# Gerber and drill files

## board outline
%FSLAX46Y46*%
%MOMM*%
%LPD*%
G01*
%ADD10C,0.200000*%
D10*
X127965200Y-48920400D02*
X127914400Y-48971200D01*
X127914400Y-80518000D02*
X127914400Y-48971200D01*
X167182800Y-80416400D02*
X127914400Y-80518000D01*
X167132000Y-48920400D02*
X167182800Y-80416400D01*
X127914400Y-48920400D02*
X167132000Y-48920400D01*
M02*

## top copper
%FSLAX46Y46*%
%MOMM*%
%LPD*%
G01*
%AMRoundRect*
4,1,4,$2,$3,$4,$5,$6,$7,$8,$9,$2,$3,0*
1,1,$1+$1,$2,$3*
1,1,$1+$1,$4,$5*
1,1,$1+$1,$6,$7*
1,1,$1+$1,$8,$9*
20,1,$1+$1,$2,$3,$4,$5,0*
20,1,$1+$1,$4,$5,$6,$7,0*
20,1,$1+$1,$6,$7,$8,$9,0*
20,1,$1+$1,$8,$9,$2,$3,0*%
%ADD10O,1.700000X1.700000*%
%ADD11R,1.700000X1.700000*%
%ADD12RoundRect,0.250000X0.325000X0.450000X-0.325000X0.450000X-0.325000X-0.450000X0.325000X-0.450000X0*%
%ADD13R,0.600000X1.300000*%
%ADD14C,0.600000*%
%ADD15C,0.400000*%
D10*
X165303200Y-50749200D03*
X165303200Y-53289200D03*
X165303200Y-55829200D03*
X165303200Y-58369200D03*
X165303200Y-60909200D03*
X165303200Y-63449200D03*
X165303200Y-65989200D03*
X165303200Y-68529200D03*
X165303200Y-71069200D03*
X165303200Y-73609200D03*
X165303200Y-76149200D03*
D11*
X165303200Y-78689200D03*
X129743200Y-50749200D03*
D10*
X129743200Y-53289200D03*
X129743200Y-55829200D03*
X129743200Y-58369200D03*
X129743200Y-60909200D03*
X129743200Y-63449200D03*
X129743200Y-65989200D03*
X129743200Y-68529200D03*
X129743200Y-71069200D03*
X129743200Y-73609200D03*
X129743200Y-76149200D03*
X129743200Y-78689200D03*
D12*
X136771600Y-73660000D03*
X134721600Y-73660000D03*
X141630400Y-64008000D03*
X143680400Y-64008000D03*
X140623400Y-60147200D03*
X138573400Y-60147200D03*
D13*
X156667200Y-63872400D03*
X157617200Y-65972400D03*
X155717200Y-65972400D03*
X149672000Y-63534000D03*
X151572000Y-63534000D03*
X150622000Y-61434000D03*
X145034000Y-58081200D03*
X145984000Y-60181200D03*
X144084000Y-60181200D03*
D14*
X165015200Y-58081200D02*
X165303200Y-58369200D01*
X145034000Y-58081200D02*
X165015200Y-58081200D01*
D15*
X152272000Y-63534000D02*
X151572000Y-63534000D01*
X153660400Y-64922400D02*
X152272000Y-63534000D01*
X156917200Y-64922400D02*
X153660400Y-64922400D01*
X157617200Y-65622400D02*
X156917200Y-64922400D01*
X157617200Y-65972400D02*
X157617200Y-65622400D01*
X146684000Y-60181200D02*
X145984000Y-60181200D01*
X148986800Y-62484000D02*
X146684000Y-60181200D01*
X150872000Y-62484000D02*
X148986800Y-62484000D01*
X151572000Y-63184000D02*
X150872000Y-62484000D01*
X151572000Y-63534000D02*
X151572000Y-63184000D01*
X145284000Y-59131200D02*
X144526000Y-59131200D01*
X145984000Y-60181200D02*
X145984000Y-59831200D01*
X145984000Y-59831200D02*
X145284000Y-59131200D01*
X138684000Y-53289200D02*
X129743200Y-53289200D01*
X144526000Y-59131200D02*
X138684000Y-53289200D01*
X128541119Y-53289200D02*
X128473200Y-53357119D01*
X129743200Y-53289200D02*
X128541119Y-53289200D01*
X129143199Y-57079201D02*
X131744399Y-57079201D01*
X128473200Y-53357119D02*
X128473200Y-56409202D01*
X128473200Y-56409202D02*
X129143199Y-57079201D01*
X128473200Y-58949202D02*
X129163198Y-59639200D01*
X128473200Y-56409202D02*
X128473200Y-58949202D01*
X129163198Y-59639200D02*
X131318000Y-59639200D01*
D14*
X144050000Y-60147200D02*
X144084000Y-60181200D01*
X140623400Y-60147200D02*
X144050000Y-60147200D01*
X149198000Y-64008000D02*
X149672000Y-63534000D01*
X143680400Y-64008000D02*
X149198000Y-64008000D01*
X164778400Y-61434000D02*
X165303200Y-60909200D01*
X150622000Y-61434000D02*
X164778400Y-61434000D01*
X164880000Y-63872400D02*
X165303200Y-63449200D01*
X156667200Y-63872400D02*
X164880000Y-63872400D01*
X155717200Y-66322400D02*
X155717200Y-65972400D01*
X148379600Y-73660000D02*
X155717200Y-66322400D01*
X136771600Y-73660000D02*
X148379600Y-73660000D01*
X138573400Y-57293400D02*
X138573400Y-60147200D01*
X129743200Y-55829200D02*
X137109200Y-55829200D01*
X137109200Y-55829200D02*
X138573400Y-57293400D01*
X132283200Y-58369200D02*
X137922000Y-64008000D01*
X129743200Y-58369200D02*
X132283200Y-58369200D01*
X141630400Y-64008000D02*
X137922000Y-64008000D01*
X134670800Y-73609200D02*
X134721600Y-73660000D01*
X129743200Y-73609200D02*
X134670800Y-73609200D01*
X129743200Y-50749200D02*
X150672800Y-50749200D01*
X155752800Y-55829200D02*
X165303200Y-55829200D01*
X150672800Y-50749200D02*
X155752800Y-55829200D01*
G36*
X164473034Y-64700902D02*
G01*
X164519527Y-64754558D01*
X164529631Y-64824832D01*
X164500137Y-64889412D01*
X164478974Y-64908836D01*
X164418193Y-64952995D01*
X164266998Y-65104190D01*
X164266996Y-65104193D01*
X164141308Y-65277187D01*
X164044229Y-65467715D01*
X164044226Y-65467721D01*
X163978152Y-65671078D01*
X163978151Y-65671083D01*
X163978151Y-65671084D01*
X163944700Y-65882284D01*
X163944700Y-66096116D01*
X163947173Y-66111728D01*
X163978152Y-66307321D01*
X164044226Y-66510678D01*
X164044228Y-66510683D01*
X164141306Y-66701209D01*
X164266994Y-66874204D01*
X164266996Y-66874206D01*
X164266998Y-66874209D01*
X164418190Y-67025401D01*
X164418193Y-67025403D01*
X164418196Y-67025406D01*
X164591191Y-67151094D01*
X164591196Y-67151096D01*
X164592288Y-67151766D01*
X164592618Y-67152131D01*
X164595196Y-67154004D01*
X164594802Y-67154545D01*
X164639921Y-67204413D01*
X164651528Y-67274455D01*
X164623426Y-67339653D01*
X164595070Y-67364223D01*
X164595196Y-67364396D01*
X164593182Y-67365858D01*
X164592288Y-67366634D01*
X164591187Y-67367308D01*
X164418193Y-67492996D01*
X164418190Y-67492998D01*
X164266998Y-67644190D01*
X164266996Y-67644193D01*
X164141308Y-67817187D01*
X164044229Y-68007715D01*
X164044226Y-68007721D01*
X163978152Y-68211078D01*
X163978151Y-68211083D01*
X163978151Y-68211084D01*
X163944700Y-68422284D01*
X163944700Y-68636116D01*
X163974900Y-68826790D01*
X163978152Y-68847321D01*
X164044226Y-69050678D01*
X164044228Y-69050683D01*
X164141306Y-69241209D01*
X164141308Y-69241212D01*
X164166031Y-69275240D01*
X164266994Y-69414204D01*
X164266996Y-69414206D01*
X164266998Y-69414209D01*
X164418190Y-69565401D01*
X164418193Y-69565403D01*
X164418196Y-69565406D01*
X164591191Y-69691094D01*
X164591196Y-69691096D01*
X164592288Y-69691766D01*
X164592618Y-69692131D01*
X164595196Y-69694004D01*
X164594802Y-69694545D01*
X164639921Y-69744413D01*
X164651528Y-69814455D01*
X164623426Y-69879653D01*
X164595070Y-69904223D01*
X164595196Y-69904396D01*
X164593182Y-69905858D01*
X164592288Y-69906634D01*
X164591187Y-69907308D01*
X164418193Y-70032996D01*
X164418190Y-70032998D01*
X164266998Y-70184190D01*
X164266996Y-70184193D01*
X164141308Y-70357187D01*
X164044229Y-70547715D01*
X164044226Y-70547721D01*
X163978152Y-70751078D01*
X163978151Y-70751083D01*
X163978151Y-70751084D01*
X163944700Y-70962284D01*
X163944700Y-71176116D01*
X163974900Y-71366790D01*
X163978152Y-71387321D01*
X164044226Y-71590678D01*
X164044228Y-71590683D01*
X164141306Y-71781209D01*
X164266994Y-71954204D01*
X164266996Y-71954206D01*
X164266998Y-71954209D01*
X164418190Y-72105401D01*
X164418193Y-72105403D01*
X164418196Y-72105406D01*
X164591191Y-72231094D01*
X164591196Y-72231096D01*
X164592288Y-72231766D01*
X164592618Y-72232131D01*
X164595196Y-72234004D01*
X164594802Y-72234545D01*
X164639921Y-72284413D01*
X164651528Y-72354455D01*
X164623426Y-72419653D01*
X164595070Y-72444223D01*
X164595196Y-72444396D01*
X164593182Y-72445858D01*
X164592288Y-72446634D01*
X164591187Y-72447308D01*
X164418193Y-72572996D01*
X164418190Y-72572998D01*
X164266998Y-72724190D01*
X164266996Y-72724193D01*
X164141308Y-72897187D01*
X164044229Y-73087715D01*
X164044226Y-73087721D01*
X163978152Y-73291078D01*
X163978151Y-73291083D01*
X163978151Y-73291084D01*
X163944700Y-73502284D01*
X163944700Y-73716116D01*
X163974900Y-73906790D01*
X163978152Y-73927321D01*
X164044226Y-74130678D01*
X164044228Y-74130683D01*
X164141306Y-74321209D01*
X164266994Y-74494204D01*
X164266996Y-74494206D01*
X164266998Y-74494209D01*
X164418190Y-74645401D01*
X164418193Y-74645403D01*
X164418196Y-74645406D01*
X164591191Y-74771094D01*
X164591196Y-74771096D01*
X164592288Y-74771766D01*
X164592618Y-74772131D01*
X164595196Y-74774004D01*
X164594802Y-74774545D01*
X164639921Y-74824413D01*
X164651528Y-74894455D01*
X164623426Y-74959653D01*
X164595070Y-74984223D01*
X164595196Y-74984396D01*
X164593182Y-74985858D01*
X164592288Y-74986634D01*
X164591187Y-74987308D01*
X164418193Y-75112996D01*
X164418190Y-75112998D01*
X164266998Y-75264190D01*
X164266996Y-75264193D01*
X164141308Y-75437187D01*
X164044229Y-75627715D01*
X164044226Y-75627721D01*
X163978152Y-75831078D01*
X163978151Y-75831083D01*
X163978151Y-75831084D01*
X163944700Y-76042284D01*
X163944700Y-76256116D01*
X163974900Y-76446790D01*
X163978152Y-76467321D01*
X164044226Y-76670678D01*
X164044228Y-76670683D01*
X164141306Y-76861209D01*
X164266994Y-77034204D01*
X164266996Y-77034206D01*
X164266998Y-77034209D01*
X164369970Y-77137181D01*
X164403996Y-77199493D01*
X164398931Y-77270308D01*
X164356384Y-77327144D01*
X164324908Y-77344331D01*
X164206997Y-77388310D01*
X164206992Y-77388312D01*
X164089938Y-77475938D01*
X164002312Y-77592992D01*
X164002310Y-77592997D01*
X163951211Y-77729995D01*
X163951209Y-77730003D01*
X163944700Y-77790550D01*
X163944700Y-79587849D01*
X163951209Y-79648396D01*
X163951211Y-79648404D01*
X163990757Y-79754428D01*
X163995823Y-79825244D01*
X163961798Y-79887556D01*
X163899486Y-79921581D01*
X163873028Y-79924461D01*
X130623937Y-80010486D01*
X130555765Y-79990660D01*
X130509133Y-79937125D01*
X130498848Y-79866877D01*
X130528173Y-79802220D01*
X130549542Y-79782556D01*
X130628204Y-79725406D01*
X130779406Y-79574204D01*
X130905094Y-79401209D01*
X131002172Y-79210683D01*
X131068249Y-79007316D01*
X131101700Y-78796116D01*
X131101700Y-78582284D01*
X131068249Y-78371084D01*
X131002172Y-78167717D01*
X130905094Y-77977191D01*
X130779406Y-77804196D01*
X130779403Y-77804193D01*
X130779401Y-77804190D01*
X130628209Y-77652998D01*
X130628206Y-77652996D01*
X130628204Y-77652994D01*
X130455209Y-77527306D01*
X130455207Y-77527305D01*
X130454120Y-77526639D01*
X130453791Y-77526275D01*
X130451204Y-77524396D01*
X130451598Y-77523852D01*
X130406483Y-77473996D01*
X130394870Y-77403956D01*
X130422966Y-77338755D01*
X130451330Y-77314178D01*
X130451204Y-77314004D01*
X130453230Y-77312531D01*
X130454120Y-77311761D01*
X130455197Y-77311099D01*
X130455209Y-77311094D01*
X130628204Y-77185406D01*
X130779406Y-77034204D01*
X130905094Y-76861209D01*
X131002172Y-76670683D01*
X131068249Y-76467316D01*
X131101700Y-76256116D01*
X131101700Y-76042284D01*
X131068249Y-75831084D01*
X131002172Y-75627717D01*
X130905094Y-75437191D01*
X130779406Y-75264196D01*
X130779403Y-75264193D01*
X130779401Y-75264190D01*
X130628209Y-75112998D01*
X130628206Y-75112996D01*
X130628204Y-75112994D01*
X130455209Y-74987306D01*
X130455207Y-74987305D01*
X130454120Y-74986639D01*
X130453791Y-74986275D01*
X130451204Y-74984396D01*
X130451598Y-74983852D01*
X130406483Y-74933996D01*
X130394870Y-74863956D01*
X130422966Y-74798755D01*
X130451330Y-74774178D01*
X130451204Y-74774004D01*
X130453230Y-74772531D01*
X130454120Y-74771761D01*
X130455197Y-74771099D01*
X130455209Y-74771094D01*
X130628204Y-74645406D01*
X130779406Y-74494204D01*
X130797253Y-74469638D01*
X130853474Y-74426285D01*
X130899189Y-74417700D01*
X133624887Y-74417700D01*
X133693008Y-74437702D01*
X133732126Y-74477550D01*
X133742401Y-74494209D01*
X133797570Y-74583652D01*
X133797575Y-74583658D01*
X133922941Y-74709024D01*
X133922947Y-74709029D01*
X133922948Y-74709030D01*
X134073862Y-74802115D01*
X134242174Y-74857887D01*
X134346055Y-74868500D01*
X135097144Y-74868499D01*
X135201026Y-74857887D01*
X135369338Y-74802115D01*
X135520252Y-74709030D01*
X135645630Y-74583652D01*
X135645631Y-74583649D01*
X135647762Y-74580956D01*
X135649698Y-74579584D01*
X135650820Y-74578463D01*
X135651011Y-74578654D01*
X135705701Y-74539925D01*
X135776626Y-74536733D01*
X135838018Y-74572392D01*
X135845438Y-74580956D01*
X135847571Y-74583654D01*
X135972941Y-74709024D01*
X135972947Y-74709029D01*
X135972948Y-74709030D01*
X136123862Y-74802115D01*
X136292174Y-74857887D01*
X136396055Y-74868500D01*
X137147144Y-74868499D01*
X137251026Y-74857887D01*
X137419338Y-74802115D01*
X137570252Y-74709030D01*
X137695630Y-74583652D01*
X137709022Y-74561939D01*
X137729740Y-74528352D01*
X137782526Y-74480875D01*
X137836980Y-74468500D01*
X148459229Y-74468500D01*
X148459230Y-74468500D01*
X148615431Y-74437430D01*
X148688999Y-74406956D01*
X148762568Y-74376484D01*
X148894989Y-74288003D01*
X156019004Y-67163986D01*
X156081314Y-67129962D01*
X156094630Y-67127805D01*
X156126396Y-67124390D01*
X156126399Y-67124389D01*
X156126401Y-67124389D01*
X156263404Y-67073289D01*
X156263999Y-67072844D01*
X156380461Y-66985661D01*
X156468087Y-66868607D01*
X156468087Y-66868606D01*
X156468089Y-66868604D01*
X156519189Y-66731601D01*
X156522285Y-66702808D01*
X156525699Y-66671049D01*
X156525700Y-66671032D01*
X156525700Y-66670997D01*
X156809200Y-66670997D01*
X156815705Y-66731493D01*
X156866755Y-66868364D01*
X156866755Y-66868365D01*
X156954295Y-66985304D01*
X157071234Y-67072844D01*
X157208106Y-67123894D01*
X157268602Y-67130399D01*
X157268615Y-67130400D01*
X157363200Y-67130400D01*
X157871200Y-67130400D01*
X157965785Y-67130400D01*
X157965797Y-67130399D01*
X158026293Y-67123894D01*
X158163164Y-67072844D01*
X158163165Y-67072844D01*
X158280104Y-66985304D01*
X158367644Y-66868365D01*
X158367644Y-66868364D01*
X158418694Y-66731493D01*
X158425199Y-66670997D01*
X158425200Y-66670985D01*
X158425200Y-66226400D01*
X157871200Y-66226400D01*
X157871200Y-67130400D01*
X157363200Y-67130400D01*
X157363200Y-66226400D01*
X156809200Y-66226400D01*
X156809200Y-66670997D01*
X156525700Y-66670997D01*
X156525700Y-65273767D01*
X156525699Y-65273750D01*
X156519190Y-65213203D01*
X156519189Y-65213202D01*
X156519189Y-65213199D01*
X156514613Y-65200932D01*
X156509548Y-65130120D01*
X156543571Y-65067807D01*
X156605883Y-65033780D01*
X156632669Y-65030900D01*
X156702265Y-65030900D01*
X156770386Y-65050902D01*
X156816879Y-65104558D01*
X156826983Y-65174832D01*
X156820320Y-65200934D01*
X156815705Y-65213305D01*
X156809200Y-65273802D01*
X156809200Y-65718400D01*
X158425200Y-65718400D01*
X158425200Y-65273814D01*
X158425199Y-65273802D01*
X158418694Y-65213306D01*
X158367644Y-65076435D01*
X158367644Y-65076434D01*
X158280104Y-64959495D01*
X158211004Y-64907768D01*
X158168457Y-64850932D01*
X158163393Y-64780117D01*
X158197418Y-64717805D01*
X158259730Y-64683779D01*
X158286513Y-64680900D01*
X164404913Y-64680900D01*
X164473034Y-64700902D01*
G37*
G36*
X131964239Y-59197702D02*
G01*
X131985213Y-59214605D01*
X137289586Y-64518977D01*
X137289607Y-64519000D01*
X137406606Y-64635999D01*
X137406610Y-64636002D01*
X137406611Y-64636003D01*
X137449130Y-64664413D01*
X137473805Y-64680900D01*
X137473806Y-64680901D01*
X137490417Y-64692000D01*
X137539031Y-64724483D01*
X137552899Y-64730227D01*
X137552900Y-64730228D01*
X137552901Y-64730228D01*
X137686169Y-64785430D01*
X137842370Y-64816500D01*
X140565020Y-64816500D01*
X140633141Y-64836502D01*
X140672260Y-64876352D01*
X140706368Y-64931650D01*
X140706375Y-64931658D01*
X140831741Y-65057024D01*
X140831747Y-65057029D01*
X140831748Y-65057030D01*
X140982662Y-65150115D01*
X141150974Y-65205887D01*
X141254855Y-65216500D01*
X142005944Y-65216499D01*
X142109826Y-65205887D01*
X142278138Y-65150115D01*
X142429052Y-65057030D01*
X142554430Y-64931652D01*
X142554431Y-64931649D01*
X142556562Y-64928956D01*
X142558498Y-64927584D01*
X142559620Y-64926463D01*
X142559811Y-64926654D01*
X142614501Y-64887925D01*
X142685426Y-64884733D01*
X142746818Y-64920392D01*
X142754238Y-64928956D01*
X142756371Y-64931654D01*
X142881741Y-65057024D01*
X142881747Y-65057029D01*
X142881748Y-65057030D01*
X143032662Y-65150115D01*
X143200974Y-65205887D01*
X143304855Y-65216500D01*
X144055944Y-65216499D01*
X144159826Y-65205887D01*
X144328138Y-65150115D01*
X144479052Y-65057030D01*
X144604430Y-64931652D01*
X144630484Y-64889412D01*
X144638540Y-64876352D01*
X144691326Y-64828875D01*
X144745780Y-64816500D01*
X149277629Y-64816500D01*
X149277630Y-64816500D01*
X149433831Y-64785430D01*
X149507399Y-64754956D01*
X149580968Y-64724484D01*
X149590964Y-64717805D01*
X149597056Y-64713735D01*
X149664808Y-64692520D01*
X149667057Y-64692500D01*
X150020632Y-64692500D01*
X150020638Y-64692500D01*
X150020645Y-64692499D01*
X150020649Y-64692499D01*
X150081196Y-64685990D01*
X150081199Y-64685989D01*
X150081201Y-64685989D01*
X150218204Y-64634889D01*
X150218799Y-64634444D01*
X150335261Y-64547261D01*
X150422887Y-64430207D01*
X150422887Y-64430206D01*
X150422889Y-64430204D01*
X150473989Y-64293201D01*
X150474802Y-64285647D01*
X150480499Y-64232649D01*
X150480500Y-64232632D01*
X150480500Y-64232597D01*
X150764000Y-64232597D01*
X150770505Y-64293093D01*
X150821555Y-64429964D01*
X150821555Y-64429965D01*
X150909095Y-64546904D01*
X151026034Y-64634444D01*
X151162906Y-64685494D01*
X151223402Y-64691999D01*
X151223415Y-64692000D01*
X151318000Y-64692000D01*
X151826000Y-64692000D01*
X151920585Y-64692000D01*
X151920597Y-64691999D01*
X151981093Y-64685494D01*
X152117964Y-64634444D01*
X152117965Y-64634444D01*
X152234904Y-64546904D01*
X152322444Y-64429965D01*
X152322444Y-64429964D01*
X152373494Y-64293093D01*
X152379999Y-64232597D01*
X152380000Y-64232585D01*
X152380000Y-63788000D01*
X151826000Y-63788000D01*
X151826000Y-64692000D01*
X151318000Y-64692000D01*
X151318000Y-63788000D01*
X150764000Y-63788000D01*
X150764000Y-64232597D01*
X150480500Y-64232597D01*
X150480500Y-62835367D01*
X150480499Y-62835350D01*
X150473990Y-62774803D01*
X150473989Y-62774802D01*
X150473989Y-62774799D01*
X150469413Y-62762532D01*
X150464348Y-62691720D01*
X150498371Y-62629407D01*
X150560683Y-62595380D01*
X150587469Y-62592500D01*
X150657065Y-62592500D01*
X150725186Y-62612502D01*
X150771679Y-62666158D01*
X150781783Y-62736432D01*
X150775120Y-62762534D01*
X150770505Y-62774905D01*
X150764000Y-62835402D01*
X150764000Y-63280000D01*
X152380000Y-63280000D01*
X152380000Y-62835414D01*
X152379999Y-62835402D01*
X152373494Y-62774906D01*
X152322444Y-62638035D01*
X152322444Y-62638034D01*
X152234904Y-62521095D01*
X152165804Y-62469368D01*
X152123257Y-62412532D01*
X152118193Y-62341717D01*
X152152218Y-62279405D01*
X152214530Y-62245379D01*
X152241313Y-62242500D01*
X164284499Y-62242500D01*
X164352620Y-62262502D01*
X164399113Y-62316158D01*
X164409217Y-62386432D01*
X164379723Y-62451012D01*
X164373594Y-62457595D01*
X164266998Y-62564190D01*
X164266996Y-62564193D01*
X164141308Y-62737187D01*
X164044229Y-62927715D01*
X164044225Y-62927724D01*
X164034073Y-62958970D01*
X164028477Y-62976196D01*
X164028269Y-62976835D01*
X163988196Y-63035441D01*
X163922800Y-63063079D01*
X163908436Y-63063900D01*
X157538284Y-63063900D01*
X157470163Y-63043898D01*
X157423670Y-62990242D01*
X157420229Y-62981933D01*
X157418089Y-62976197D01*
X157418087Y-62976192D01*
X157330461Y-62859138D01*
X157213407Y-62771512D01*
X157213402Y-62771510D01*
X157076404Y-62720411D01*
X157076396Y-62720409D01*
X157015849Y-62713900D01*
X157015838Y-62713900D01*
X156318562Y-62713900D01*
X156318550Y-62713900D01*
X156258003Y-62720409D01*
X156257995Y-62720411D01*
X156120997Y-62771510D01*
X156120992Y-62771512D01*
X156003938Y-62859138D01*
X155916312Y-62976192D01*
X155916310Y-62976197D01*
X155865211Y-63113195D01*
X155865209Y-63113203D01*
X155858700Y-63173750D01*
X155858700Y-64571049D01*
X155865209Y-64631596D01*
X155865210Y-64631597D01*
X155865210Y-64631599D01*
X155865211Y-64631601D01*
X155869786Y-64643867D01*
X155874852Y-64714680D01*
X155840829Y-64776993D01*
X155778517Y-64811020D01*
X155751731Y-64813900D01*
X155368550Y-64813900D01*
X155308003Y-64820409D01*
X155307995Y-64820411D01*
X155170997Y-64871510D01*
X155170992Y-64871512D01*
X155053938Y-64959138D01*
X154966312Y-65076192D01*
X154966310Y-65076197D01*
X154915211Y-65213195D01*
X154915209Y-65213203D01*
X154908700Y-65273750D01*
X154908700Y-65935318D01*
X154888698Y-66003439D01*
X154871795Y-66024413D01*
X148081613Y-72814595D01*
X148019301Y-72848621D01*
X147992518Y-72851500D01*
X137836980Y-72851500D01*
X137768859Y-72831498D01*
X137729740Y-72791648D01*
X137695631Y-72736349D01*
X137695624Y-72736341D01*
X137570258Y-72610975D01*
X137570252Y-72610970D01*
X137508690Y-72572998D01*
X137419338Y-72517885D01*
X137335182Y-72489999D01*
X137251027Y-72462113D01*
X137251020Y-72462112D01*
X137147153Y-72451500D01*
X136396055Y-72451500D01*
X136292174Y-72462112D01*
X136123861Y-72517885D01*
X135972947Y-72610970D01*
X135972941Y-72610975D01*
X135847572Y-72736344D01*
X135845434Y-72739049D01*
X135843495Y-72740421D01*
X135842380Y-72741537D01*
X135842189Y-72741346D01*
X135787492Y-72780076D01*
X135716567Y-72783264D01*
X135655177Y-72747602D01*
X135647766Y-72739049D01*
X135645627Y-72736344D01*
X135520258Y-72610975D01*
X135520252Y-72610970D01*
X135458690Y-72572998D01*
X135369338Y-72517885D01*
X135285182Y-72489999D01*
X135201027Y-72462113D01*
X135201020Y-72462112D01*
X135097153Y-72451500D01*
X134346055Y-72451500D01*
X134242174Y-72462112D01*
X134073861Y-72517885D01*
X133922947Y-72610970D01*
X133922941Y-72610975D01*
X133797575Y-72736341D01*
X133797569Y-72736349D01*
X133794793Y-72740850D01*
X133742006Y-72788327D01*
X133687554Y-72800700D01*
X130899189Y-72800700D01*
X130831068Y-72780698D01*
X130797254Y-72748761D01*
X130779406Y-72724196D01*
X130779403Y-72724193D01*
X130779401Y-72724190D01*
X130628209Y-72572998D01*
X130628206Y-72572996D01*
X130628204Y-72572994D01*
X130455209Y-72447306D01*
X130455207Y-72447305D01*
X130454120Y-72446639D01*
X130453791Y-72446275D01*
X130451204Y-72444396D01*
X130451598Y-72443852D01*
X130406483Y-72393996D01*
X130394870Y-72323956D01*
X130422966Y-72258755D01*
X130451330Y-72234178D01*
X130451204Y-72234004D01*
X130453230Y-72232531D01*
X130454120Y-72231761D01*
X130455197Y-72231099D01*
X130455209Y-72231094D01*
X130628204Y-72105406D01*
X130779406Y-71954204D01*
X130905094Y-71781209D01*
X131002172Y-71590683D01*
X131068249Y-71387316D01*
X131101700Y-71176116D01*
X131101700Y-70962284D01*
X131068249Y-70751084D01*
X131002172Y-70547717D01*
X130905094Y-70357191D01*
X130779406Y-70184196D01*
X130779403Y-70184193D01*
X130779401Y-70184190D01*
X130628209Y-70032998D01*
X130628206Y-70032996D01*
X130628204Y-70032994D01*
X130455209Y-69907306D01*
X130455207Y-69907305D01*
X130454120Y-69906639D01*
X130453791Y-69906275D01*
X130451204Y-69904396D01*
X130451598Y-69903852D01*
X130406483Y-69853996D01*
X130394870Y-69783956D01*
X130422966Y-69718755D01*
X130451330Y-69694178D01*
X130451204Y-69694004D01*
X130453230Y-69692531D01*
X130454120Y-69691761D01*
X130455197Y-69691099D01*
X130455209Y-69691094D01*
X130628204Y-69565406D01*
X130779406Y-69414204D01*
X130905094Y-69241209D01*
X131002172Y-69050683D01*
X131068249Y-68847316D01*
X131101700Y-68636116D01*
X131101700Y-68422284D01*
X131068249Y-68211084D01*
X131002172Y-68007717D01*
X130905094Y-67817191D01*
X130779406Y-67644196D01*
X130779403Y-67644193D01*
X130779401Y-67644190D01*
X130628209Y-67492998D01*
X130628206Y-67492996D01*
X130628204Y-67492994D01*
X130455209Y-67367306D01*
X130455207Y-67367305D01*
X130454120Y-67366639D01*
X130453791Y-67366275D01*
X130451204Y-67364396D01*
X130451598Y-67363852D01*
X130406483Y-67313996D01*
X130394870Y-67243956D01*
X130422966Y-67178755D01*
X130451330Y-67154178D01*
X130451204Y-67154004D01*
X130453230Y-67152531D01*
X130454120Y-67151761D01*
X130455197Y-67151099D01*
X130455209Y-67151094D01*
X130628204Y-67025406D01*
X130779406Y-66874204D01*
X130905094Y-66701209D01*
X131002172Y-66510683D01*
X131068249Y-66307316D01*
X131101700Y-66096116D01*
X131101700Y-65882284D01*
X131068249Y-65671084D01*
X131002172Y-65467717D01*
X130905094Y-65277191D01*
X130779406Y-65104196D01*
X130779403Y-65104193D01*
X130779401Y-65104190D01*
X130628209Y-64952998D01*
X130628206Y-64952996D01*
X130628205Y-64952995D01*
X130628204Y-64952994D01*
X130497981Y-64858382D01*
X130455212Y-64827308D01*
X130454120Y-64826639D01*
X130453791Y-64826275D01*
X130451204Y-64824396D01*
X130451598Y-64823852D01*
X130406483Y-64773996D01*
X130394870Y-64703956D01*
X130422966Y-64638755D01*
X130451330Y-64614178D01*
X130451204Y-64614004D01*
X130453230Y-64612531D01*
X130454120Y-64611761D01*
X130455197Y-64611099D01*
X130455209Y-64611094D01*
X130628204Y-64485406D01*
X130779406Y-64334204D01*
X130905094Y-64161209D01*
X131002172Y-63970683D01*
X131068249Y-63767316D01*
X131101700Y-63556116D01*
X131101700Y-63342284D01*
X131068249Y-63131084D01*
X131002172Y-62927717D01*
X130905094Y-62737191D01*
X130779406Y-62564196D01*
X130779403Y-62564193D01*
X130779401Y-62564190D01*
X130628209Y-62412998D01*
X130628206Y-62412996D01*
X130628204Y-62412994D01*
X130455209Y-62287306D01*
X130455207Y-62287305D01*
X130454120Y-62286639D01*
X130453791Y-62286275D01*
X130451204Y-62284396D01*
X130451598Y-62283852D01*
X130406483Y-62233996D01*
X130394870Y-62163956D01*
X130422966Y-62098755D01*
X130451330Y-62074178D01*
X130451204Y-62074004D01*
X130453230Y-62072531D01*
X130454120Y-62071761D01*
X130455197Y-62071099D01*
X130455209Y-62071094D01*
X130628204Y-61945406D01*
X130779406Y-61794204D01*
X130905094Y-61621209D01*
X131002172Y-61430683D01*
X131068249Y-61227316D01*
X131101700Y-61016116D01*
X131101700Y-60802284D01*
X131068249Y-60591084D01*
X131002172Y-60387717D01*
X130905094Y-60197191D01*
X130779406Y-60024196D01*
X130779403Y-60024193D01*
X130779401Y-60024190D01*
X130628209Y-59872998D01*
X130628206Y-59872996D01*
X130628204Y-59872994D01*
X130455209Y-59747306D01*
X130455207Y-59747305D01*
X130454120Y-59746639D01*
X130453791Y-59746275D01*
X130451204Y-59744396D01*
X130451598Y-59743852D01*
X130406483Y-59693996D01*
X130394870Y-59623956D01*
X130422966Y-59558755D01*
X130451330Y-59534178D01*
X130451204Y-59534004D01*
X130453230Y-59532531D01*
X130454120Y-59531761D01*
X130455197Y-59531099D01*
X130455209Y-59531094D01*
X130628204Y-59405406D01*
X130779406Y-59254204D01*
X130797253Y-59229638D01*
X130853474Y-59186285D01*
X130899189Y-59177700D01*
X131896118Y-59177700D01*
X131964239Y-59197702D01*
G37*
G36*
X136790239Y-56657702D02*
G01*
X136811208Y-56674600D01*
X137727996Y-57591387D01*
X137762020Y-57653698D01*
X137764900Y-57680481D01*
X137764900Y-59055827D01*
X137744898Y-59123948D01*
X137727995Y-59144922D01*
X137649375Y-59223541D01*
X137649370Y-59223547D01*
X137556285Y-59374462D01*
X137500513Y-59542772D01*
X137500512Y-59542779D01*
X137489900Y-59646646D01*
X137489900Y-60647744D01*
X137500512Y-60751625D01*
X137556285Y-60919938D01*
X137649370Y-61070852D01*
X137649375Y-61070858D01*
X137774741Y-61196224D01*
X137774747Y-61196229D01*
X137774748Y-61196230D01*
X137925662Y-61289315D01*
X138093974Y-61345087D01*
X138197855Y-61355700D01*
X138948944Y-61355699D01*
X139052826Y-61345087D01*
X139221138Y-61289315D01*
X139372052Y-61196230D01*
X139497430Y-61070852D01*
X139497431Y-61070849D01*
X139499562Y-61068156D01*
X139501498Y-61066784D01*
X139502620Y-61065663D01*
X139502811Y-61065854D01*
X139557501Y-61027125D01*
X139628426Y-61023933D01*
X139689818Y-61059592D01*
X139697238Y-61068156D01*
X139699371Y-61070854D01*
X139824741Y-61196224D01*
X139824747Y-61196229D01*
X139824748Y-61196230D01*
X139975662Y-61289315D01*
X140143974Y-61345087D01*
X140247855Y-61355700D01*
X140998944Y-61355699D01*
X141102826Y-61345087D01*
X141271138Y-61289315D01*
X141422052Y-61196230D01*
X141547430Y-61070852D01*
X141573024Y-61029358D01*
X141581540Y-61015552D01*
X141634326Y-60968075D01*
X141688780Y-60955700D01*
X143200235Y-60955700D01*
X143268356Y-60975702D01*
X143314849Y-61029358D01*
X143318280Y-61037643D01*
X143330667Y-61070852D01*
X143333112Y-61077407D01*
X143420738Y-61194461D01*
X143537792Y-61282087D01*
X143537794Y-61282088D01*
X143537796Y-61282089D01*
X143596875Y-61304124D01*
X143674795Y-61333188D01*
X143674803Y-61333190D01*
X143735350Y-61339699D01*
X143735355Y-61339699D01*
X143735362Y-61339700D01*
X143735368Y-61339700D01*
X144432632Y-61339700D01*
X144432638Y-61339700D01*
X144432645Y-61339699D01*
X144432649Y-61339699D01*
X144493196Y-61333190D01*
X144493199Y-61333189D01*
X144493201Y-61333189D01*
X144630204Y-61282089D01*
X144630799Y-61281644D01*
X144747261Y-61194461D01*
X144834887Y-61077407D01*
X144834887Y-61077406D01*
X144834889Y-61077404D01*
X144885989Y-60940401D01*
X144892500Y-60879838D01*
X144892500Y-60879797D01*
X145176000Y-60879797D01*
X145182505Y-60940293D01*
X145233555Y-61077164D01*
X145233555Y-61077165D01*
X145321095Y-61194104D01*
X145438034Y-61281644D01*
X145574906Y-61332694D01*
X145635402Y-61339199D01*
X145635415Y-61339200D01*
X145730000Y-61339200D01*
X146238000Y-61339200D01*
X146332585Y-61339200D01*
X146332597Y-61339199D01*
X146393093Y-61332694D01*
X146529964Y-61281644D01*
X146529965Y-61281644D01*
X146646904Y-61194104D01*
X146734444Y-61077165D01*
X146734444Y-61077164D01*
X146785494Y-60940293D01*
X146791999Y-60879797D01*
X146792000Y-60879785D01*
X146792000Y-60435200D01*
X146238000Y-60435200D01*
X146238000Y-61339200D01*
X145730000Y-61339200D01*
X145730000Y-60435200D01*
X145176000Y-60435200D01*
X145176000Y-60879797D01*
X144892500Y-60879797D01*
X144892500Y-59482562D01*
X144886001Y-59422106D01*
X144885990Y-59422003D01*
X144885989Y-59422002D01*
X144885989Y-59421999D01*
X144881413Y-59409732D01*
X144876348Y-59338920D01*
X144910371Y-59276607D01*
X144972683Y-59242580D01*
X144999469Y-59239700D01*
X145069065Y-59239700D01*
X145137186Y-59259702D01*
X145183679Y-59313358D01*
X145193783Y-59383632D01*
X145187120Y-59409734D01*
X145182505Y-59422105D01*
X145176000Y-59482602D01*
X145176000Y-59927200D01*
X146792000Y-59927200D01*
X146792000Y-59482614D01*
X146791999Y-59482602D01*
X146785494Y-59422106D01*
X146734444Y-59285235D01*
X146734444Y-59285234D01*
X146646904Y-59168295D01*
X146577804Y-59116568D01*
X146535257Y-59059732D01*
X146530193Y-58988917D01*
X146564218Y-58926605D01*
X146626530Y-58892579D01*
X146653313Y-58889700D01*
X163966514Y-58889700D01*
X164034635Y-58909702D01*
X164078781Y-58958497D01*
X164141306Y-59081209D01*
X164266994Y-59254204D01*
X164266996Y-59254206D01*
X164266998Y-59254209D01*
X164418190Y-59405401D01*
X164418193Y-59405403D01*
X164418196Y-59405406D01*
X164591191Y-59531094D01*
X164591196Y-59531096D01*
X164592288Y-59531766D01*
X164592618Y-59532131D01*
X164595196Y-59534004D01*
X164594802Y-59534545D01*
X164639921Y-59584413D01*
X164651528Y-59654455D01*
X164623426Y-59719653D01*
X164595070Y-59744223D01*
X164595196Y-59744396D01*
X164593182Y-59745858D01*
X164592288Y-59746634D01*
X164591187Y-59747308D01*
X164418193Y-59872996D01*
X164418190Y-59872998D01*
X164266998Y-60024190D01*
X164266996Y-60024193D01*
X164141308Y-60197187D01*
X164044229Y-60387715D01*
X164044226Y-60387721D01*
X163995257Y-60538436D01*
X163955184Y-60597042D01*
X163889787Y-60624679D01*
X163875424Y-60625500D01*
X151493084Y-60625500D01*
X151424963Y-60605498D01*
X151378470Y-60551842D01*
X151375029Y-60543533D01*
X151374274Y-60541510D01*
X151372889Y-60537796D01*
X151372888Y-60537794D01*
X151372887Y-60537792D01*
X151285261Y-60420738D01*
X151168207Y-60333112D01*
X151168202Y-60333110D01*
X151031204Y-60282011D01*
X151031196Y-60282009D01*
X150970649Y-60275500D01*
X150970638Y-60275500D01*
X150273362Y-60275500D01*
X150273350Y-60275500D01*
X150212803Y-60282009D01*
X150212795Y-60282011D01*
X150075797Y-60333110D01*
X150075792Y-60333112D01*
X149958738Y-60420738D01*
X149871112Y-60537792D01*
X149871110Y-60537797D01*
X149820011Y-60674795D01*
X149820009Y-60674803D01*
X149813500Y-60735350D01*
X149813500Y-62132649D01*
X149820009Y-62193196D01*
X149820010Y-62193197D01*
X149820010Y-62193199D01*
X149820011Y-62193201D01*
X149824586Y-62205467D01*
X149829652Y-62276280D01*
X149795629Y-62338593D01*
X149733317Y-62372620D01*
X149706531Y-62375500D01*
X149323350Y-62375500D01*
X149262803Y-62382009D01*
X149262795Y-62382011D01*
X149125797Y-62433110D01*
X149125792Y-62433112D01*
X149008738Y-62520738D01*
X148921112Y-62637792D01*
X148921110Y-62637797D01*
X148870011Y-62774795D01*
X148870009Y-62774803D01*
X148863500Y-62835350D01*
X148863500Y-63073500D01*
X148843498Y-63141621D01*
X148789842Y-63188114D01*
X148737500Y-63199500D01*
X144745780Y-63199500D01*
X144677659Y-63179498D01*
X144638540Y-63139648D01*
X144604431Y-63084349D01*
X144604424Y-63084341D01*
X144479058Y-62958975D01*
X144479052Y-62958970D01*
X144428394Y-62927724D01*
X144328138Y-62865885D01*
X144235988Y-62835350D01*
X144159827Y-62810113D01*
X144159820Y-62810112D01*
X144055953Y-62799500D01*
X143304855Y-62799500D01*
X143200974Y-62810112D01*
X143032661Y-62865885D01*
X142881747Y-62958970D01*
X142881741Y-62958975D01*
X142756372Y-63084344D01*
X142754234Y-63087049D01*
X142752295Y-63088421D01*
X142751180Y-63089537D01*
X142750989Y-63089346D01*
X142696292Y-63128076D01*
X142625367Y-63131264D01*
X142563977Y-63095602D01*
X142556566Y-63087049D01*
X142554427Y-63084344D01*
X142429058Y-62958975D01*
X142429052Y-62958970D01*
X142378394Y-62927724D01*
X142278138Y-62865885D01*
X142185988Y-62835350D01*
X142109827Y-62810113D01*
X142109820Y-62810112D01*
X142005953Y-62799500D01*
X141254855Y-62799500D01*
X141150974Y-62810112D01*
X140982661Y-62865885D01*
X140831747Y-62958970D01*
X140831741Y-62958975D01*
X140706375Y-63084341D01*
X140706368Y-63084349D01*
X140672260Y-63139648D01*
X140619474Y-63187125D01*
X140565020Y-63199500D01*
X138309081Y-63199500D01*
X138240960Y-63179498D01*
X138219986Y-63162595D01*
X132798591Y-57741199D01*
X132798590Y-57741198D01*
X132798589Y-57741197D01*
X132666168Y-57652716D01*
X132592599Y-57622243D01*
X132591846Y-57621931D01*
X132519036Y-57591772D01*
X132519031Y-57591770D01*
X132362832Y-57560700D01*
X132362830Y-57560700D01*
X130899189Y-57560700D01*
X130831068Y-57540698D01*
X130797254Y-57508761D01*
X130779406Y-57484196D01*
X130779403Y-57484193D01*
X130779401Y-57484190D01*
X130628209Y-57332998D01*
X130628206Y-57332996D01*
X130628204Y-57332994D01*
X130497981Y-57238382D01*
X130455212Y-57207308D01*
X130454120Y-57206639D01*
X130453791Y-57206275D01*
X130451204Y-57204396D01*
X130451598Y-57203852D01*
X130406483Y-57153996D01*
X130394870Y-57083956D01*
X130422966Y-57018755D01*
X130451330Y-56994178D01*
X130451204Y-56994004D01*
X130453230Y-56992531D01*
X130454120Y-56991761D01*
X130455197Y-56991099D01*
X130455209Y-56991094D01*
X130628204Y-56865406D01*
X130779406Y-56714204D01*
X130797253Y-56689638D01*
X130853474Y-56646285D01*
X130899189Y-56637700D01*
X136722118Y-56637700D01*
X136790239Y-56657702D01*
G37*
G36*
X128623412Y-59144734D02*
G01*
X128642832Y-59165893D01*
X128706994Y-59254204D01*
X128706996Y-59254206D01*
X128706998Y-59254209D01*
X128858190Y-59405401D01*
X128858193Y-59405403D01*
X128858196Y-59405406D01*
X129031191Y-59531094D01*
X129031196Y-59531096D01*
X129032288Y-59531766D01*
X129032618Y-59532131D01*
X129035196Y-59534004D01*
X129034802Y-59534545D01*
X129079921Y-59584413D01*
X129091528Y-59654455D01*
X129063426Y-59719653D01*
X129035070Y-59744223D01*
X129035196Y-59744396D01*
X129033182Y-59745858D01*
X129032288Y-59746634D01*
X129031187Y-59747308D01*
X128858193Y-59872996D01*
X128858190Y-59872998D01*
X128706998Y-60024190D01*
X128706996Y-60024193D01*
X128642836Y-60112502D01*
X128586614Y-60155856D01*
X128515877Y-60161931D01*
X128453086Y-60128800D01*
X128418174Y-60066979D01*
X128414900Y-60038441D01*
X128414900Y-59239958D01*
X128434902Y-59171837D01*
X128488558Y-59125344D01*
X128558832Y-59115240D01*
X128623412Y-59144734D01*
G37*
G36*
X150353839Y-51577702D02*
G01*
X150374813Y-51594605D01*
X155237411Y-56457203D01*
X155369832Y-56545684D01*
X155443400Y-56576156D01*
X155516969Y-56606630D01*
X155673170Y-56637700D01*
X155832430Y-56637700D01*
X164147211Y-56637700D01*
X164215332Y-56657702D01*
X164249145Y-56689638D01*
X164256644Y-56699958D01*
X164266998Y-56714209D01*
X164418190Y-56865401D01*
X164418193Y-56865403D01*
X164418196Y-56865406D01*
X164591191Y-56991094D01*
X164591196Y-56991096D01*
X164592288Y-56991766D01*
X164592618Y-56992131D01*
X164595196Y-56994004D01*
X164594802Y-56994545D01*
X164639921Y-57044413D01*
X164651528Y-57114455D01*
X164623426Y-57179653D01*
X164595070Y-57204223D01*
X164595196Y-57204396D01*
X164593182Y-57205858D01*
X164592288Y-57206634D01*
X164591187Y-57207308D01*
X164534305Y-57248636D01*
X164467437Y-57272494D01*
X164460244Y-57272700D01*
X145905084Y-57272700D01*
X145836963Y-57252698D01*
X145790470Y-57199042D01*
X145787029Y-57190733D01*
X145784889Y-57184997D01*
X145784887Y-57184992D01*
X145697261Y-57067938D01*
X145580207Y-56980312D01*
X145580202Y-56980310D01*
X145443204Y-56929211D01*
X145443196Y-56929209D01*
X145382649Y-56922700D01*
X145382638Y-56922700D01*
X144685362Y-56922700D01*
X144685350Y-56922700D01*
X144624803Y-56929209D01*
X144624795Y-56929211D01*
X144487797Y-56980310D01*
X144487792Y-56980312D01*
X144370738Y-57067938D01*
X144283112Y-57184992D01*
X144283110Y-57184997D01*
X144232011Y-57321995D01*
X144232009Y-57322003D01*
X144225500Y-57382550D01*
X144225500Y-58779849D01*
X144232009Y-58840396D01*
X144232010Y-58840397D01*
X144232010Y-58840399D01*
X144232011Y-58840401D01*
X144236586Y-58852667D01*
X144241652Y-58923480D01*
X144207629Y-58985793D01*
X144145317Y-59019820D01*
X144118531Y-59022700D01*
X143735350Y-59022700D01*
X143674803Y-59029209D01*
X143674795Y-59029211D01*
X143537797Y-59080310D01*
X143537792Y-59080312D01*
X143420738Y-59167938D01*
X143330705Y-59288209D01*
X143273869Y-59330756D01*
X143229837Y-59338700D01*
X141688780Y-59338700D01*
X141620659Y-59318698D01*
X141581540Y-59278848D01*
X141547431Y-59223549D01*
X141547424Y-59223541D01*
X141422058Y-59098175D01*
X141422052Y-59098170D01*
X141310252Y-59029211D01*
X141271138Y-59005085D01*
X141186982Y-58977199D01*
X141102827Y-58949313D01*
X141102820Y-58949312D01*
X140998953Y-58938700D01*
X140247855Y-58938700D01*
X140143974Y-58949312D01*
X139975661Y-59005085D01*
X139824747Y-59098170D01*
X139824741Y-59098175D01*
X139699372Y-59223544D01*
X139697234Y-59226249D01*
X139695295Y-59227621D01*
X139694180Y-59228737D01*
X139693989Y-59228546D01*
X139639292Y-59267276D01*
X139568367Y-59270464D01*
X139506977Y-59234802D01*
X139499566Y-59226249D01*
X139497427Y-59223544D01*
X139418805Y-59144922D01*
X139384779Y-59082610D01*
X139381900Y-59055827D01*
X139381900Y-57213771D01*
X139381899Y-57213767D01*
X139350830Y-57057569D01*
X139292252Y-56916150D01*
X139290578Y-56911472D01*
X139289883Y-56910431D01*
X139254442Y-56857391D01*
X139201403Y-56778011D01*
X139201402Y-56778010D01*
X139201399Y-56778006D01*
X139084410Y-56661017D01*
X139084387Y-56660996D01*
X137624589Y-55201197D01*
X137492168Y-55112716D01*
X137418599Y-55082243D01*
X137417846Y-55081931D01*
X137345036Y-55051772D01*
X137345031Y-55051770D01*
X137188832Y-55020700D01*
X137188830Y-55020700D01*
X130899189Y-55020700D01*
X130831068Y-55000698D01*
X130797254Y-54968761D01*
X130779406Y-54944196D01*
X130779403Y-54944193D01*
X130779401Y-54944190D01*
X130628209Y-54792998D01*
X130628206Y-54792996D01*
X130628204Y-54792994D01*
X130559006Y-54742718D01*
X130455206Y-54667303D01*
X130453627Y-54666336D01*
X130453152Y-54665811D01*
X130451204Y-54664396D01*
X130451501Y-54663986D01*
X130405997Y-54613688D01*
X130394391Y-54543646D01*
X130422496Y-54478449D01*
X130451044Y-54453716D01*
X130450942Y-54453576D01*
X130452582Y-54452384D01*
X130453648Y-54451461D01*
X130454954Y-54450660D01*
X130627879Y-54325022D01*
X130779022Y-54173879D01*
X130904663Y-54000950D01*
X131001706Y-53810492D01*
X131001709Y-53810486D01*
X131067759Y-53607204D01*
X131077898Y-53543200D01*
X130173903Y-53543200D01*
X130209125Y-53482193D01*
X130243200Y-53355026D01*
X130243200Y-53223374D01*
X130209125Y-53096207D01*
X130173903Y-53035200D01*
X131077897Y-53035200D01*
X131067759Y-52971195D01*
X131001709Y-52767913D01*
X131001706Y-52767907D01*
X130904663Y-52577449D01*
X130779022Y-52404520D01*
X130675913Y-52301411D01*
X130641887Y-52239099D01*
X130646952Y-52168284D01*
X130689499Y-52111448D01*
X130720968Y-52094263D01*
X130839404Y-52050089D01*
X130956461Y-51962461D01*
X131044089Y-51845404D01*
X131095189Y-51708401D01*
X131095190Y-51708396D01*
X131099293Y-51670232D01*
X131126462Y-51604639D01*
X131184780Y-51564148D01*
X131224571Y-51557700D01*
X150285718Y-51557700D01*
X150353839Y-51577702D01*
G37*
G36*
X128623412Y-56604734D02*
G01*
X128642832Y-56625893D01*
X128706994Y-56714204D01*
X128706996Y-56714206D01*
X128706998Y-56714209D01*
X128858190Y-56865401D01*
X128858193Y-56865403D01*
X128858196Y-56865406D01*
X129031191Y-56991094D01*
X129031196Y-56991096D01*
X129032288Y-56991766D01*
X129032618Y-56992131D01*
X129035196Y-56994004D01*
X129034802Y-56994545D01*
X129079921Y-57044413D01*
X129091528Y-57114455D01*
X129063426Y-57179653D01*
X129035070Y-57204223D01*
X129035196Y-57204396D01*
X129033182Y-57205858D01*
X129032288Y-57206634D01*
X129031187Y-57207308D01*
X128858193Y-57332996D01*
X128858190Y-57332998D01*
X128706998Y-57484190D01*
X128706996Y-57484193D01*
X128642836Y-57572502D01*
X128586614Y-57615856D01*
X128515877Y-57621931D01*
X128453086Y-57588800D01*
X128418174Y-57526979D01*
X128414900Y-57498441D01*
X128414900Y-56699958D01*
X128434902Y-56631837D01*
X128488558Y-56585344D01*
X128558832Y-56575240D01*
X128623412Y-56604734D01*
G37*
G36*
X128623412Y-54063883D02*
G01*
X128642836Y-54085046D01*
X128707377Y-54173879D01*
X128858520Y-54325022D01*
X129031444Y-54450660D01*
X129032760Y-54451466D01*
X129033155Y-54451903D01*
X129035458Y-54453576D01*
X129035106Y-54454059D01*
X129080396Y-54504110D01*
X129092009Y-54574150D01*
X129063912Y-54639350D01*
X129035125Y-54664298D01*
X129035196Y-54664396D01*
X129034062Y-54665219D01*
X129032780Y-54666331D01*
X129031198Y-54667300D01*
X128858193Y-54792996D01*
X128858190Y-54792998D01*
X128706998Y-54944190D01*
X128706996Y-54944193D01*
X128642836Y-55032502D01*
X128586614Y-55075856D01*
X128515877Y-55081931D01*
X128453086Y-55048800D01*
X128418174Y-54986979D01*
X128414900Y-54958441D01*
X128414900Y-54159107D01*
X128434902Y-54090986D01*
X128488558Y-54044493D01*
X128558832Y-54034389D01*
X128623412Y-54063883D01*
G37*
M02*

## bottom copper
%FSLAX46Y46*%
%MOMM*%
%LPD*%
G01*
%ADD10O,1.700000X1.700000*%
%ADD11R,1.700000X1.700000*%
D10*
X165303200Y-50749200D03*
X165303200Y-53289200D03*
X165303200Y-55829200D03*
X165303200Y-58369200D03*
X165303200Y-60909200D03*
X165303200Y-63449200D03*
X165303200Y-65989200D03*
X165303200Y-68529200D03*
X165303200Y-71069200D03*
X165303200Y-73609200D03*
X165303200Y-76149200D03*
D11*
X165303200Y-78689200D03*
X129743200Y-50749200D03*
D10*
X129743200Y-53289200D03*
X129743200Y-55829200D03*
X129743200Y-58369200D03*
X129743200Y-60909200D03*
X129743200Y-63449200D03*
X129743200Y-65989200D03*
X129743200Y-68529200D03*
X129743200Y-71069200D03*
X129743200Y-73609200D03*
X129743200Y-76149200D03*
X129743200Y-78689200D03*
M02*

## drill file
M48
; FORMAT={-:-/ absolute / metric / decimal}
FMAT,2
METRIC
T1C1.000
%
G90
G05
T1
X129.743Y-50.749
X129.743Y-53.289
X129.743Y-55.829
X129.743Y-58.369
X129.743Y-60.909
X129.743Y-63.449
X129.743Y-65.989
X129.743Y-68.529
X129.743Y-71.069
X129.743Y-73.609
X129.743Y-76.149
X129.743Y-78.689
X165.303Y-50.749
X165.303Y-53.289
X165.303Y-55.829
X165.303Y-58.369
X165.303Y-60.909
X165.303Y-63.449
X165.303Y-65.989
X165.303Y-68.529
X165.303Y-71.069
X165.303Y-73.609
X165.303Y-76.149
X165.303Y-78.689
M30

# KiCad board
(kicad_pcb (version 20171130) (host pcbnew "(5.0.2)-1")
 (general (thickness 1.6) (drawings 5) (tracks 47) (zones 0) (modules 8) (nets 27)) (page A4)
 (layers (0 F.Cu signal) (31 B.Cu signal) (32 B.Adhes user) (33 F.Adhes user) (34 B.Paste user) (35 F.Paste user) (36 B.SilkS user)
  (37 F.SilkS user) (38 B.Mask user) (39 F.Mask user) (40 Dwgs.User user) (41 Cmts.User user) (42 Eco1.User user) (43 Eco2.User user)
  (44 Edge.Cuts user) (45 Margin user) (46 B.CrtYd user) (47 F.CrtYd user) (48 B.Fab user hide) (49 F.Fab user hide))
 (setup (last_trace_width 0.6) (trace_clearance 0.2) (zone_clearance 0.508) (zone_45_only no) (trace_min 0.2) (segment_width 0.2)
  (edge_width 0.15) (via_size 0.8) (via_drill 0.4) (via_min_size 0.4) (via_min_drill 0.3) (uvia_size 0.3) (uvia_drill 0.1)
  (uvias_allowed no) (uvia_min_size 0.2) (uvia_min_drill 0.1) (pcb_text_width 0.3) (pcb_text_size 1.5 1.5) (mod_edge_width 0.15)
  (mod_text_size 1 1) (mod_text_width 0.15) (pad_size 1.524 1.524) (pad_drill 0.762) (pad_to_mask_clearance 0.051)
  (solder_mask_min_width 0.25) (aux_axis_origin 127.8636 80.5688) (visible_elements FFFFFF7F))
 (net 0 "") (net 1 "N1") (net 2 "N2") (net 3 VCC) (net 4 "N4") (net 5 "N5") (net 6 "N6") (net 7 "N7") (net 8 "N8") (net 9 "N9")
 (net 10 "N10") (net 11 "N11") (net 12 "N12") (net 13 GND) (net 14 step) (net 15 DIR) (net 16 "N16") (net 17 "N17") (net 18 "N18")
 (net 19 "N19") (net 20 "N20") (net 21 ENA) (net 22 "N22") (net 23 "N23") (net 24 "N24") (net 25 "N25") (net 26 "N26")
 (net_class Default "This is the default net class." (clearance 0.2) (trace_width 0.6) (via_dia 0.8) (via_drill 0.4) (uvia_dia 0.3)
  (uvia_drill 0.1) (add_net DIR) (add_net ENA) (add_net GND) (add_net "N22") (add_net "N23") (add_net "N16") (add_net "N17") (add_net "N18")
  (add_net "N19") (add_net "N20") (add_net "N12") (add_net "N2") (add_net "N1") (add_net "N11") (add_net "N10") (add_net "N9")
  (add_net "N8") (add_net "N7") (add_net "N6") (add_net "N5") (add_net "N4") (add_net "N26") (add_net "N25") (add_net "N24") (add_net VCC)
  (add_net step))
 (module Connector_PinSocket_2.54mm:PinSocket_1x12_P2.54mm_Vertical (layer F.Cu) (at 165.3032 78.6892 180)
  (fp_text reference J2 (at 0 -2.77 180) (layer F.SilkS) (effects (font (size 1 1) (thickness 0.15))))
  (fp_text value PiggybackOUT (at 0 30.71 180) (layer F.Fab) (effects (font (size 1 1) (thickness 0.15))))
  (pad 12 thru_hole oval (at 0 27.94 180) (size 1.7 1.7) (drill 1) (layers *.Cu *.Mask) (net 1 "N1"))
  (pad 11 thru_hole oval (at 0 25.4 180) (size 1.7 1.7) (drill 1) (layers *.Cu *.Mask) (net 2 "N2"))
  (pad 10 thru_hole oval (at 0 22.86 180) (size 1.7 1.7) (drill 1) (layers *.Cu *.Mask) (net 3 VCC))
  (pad 9 thru_hole oval (at 0 20.32 180) (size 1.7 1.7) (drill 1) (layers *.Cu *.Mask) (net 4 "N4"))
  (pad 8 thru_hole oval (at 0 17.78 180) (size 1.7 1.7) (drill 1) (layers *.Cu *.Mask) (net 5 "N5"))
  (pad 7 thru_hole oval (at 0 15.24 180) (size 1.7 1.7) (drill 1) (layers *.Cu *.Mask) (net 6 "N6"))
  (pad 6 thru_hole oval (at 0 12.7 180) (size 1.7 1.7) (drill 1) (layers *.Cu *.Mask) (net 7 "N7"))
  (pad 5 thru_hole oval (at 0 10.16 180) (size 1.7 1.7) (drill 1) (layers *.Cu *.Mask) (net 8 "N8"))
  (pad 4 thru_hole oval (at 0 7.62 180) (size 1.7 1.7) (drill 1) (layers *.Cu *.Mask) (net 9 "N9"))
  (pad 3 thru_hole oval (at 0 5.08 180) (size 1.7 1.7) (drill 1) (layers *.Cu *.Mask) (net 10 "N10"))
  (pad 2 thru_hole oval (at 0 2.54 180) (size 1.7 1.7) (drill 1) (layers *.Cu *.Mask) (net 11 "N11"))
  (pad 1 thru_hole rect (at 0 0 180) (size 1.7 1.7) (drill 1) (layers *.Cu *.Mask) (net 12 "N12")))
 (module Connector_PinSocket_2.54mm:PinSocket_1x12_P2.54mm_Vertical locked (layer F.Cu) (at 129.7432 50.7492)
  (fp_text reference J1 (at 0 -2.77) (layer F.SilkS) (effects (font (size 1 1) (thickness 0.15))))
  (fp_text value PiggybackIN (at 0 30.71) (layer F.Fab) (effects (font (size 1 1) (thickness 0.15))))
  (pad 1 thru_hole rect (at 0 0) (size 1.7 1.7) (drill 1) (layers *.Cu *.Mask) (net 3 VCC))
  (pad 2 thru_hole oval (at 0 2.54) (size 1.7 1.7) (drill 1) (layers *.Cu *.Mask) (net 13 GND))
  (pad 3 thru_hole oval (at 0 5.08) (size 1.7 1.7) (drill 1) (layers *.Cu *.Mask) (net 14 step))
  (pad 4 thru_hole oval (at 0 7.62) (size 1.7 1.7) (drill 1) (layers *.Cu *.Mask) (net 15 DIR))
  (pad 5 thru_hole oval (at 0 10.16) (size 1.7 1.7) (drill 1) (layers *.Cu *.Mask) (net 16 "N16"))
  (pad 6 thru_hole oval (at 0 12.7) (size 1.7 1.7) (drill 1) (layers *.Cu *.Mask) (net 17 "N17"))
  (pad 7 thru_hole oval (at 0 15.24) (size 1.7 1.7) (drill 1) (layers *.Cu *.Mask) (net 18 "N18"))
  (pad 8 thru_hole oval (at 0 17.78) (size 1.7 1.7) (drill 1) (layers *.Cu *.Mask) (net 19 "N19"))
  (pad 9 thru_hole oval (at 0 20.32) (size 1.7 1.7) (drill 1) (layers *.Cu *.Mask) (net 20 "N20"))
  (pad 10 thru_hole oval (at 0 22.86) (size 1.7 1.7) (drill 1) (layers *.Cu *.Mask) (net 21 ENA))
  (pad 11 thru_hole oval (at 0 25.4) (size 1.7 1.7) (drill 1) (layers *.Cu *.Mask) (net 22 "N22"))
  (pad 12 thru_hole oval (at 0 27.94) (size 1.7 1.7) (drill 1) (layers *.Cu *.Mask) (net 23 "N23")))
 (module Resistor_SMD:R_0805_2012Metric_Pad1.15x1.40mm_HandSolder (layer F.Cu) (at 135.7466 73.66 180)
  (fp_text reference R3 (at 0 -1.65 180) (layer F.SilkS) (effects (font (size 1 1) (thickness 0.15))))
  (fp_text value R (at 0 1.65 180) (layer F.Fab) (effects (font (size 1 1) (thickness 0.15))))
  (pad 1 smd roundrect (at -1.025 0 180) (size 1.15 1.4) (layers F.Cu F.Paste F.Mask) (roundrect_rratio 0.217391) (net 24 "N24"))
  (pad 2 smd roundrect (at 1.025 0 180) (size 1.15 1.4) (layers F.Cu F.Paste F.Mask) (roundrect_rratio 0.217391) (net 21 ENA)))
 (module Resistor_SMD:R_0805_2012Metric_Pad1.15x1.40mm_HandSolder (layer F.Cu) (at 142.6554 64.008 180)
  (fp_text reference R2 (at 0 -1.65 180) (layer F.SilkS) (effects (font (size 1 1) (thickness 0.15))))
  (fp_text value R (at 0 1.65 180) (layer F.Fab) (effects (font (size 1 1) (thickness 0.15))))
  (pad 2 smd roundrect (at 1.025 0 180) (size 1.15 1.4) (layers F.Cu F.Paste F.Mask) (roundrect_rratio 0.217391) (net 15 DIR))
  (pad 1 smd roundrect (at -1.025 0 180) (size 1.15 1.4) (layers F.Cu F.Paste F.Mask) (roundrect_rratio 0.217391) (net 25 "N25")))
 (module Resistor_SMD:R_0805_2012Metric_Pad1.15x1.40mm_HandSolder (layer F.Cu) (at 139.5984 60.1472 180)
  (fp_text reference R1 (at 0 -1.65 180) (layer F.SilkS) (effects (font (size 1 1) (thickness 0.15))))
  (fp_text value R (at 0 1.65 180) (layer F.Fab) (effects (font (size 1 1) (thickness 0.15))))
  (pad 1 smd roundrect (at -1.025 0 180) (size 1.15 1.4) (layers F.Cu F.Paste F.Mask) (roundrect_rratio 0.217391) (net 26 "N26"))
  (pad 2 smd roundrect (at 1.025 0 180) (size 1.15 1.4) (layers F.Cu F.Paste F.Mask) (roundrect_rratio 0.217391) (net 14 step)))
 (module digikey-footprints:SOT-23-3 (layer F.Cu) (at 156.6672 64.9224 90)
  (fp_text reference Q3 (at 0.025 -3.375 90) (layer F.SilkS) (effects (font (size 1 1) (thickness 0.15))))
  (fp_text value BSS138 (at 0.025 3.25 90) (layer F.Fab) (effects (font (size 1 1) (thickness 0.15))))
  (pad 3 smd rect (at 1.05 0 90) (size 1.3 0.6) (layers F.Cu F.Paste F.Mask) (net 6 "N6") (solder_mask_margin 0.07))
  (pad 2 smd rect (at -1.05 0.95 90) (size 1.3 0.6) (layers F.Cu F.Paste F.Mask) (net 13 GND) (solder_mask_margin 0.07))
  (pad 1 smd rect (at -1.05 -0.95 90) (size 1.3 0.6) (layers F.Cu F.Paste F.Mask) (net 24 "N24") (solder_mask_margin 0.07)))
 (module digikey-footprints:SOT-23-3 (layer F.Cu) (at 150.622 62.484 90)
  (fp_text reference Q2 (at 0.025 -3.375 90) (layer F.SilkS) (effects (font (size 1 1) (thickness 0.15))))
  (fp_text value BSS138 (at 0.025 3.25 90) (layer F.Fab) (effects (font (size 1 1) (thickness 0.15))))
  (pad 1 smd rect (at -1.05 -0.95 90) (size 1.3 0.6) (layers F.Cu F.Paste F.Mask) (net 25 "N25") (solder_mask_margin 0.07))
  (pad 2 smd rect (at -1.05 0.95 90) (size 1.3 0.6) (layers F.Cu F.Paste F.Mask) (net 13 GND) (solder_mask_margin 0.07))
  (pad 3 smd rect (at 1.05 0 90) (size 1.3 0.6) (layers F.Cu F.Paste F.Mask) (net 5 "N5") (solder_mask_margin 0.07)))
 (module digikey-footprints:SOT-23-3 (layer F.Cu) (at 145.034 59.1312 90)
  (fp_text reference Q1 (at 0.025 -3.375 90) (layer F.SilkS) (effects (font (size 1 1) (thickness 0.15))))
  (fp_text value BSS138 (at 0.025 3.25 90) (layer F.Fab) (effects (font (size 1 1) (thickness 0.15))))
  (pad 3 smd rect (at 1.05 0 90) (size 1.3 0.6) (layers F.Cu F.Paste F.Mask) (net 4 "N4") (solder_mask_margin 0.07))
  (pad 2 smd rect (at -1.05 0.95 90) (size 1.3 0.6) (layers F.Cu F.Paste F.Mask) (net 13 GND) (solder_mask_margin 0.07))
  (pad 1 smd rect (at -1.05 -0.95 90) (size 1.3 0.6) (layers F.Cu F.Paste F.Mask) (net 26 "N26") (solder_mask_margin 0.07)))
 (gr_line (start 127.9652 48.9204) (end 127.9144 48.9712) (layer Edge.Cuts) (width 0.2))
 (gr_line (start 127.9144 80.518) (end 127.9144 48.9712) (layer Edge.Cuts) (width 0.2))
 (gr_line (start 167.1828 80.4164) (end 127.9144 80.518) (layer Edge.Cuts) (width 0.2))
 (gr_line (start 167.132 48.9204) (end 167.1828 80.4164) (layer Edge.Cuts) (width 0.2))
 (gr_line (start 127.9144 48.9204) (end 167.132 48.9204) (layer Edge.Cuts) (width 0.2))
 (segment (start 165.0152 58.0812) (end 165.3032 58.3692) (width 0.6) (layer F.Cu) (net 4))
 (segment (start 145.034 58.0812) (end 165.0152 58.0812) (width 0.6) (layer F.Cu) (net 4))
 (segment (start 152.272 63.534) (end 151.572 63.534) (width 0.4) (layer F.Cu) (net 13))
 (segment (start 153.6604 64.9224) (end 152.272 63.534) (width 0.4) (layer F.Cu) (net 13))
 (segment (start 156.9172 64.9224) (end 153.6604 64.9224) (width 0.4) (layer F.Cu) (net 13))
 (segment (start 157.6172 65.6224) (end 156.9172 64.9224) (width 0.4) (layer F.Cu) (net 13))
 (segment (start 157.6172 65.9724) (end 157.6172 65.6224) (width 0.4) (layer F.Cu) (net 13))
 (segment (start 146.684 60.1812) (end 145.984 60.1812) (width 0.4) (layer F.Cu) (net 13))
 (segment (start 148.9868 62.484) (end 146.684 60.1812) (width 0.4) (layer F.Cu) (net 13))
 (segment (start 150.872 62.484) (end 148.9868 62.484) (width 0.4) (layer F.Cu) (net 13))
 (segment (start 151.572 63.184) (end 150.872 62.484) (width 0.4) (layer F.Cu) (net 13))
 (segment (start 151.572 63.534) (end 151.572 63.184) (width 0.4) (layer F.Cu) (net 13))
 (segment (start 145.284 59.1312) (end 144.526 59.1312) (width 0.4) (layer F.Cu) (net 13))
 (segment (start 145.984 60.1812) (end 145.984 59.8312) (width 0.4) (layer F.Cu) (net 13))
 (segment (start 145.984 59.8312) (end 145.284 59.1312) (width 0.4) (layer F.Cu) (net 13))
 (segment (start 138.684 53.2892) (end 129.7432 53.2892) (width 0.4) (layer F.Cu) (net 13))
 (segment (start 144.526 59.1312) (end 138.684 53.2892) (width 0.4) (layer F.Cu) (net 13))
 (segment (start 128.541119 53.2892) (end 128.4732 53.357119) (width 0.4) (layer F.Cu) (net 13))
 (segment (start 129.7432 53.2892) (end 128.541119 53.2892) (width 0.4) (layer F.Cu) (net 13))
 (segment (start 129.143199 57.079201) (end 131.744399 57.079201) (width 0.4) (layer F.Cu) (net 13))
 (segment (start 128.4732 53.357119) (end 128.4732 56.409202) (width 0.4) (layer F.Cu) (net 13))
 (segment (start 128.4732 56.409202) (end 129.143199 57.079201) (width 0.4) (layer F.Cu) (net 13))
 (segment (start 128.4732 58.949202) (end 129.163198 59.6392) (width 0.4) (layer F.Cu) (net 13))
 (segment (start 128.4732 56.409202) (end 128.4732 58.949202) (width 0.4) (layer F.Cu) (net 13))
 (segment (start 129.163198 59.6392) (end 131.318 59.6392) (width 0.4) (layer F.Cu) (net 13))
 (segment (start 144.05 60.1472) (end 144.084 60.1812) (width 0.6) (layer F.Cu) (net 26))
 (segment (start 140.6234 60.1472) (end 144.05 60.1472) (width 0.6) (layer F.Cu) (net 26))
 (segment (start 149.198 64.008) (end 149.672 63.534) (width 0.6) (layer F.Cu) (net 25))
 (segment (start 143.6804 64.008) (end 149.198 64.008) (width 0.6) (layer F.Cu) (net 25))
 (segment (start 164.7784 61.434) (end 165.3032 60.9092) (width 0.6) (layer F.Cu) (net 5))
 (segment (start 150.622 61.434) (end 164.7784 61.434) (width 0.6) (layer F.Cu) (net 5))
 (segment (start 164.88 63.8724) (end 165.3032 63.4492) (width 0.6) (layer F.Cu) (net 6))
 (segment (start 156.6672 63.8724) (end 164.88 63.8724) (width 0.6) (layer F.Cu) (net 6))
 (segment (start 155.7172 66.3224) (end 155.7172 65.9724) (width 0.6) (layer F.Cu) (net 24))
 (segment (start 148.3796 73.66) (end 155.7172 66.3224) (width 0.6) (layer F.Cu) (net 24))
 (segment (start 136.7716 73.66) (end 148.3796 73.66) (width 0.6) (layer F.Cu) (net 24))
 (segment (start 138.5734 57.2934) (end 138.5734 60.1472) (width 0.6) (layer F.Cu) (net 14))
 (segment (start 129.7432 55.8292) (end 137.1092 55.8292) (width 0.6) (layer F.Cu) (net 14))
 (segment (start 137.1092 55.8292) (end 138.5734 57.2934) (width 0.6) (layer F.Cu) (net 14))
 (segment (start 132.2832 58.3692) (end 137.922 64.008) (width 0.6) (layer F.Cu) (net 15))
 (segment (start 129.7432 58.3692) (end 132.2832 58.3692) (width 0.6) (layer F.Cu) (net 15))
 (segment (start 141.6304 64.008) (end 137.922 64.008) (width 0.6) (layer F.Cu) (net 15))
 (segment (start 134.6708 73.6092) (end 134.7216 73.66) (width 0.6) (layer F.Cu) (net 21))
 (segment (start 129.7432 73.6092) (end 134.6708 73.6092) (width 0.6) (layer F.Cu) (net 21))
 (segment (start 129.7432 50.7492) (end 150.6728 50.7492) (width 0.6) (layer F.Cu) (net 3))
 (segment (start 155.7528 55.8292) (end 165.3032 55.8292) (width 0.6) (layer F.Cu) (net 3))
 (segment (start 150.6728 50.7492) (end 155.7528 55.8292) (width 0.6) (layer F.Cu) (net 3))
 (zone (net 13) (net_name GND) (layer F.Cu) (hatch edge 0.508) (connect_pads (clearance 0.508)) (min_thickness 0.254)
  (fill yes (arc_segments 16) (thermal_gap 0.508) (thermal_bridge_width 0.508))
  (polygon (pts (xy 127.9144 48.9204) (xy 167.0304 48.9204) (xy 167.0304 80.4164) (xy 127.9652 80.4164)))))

